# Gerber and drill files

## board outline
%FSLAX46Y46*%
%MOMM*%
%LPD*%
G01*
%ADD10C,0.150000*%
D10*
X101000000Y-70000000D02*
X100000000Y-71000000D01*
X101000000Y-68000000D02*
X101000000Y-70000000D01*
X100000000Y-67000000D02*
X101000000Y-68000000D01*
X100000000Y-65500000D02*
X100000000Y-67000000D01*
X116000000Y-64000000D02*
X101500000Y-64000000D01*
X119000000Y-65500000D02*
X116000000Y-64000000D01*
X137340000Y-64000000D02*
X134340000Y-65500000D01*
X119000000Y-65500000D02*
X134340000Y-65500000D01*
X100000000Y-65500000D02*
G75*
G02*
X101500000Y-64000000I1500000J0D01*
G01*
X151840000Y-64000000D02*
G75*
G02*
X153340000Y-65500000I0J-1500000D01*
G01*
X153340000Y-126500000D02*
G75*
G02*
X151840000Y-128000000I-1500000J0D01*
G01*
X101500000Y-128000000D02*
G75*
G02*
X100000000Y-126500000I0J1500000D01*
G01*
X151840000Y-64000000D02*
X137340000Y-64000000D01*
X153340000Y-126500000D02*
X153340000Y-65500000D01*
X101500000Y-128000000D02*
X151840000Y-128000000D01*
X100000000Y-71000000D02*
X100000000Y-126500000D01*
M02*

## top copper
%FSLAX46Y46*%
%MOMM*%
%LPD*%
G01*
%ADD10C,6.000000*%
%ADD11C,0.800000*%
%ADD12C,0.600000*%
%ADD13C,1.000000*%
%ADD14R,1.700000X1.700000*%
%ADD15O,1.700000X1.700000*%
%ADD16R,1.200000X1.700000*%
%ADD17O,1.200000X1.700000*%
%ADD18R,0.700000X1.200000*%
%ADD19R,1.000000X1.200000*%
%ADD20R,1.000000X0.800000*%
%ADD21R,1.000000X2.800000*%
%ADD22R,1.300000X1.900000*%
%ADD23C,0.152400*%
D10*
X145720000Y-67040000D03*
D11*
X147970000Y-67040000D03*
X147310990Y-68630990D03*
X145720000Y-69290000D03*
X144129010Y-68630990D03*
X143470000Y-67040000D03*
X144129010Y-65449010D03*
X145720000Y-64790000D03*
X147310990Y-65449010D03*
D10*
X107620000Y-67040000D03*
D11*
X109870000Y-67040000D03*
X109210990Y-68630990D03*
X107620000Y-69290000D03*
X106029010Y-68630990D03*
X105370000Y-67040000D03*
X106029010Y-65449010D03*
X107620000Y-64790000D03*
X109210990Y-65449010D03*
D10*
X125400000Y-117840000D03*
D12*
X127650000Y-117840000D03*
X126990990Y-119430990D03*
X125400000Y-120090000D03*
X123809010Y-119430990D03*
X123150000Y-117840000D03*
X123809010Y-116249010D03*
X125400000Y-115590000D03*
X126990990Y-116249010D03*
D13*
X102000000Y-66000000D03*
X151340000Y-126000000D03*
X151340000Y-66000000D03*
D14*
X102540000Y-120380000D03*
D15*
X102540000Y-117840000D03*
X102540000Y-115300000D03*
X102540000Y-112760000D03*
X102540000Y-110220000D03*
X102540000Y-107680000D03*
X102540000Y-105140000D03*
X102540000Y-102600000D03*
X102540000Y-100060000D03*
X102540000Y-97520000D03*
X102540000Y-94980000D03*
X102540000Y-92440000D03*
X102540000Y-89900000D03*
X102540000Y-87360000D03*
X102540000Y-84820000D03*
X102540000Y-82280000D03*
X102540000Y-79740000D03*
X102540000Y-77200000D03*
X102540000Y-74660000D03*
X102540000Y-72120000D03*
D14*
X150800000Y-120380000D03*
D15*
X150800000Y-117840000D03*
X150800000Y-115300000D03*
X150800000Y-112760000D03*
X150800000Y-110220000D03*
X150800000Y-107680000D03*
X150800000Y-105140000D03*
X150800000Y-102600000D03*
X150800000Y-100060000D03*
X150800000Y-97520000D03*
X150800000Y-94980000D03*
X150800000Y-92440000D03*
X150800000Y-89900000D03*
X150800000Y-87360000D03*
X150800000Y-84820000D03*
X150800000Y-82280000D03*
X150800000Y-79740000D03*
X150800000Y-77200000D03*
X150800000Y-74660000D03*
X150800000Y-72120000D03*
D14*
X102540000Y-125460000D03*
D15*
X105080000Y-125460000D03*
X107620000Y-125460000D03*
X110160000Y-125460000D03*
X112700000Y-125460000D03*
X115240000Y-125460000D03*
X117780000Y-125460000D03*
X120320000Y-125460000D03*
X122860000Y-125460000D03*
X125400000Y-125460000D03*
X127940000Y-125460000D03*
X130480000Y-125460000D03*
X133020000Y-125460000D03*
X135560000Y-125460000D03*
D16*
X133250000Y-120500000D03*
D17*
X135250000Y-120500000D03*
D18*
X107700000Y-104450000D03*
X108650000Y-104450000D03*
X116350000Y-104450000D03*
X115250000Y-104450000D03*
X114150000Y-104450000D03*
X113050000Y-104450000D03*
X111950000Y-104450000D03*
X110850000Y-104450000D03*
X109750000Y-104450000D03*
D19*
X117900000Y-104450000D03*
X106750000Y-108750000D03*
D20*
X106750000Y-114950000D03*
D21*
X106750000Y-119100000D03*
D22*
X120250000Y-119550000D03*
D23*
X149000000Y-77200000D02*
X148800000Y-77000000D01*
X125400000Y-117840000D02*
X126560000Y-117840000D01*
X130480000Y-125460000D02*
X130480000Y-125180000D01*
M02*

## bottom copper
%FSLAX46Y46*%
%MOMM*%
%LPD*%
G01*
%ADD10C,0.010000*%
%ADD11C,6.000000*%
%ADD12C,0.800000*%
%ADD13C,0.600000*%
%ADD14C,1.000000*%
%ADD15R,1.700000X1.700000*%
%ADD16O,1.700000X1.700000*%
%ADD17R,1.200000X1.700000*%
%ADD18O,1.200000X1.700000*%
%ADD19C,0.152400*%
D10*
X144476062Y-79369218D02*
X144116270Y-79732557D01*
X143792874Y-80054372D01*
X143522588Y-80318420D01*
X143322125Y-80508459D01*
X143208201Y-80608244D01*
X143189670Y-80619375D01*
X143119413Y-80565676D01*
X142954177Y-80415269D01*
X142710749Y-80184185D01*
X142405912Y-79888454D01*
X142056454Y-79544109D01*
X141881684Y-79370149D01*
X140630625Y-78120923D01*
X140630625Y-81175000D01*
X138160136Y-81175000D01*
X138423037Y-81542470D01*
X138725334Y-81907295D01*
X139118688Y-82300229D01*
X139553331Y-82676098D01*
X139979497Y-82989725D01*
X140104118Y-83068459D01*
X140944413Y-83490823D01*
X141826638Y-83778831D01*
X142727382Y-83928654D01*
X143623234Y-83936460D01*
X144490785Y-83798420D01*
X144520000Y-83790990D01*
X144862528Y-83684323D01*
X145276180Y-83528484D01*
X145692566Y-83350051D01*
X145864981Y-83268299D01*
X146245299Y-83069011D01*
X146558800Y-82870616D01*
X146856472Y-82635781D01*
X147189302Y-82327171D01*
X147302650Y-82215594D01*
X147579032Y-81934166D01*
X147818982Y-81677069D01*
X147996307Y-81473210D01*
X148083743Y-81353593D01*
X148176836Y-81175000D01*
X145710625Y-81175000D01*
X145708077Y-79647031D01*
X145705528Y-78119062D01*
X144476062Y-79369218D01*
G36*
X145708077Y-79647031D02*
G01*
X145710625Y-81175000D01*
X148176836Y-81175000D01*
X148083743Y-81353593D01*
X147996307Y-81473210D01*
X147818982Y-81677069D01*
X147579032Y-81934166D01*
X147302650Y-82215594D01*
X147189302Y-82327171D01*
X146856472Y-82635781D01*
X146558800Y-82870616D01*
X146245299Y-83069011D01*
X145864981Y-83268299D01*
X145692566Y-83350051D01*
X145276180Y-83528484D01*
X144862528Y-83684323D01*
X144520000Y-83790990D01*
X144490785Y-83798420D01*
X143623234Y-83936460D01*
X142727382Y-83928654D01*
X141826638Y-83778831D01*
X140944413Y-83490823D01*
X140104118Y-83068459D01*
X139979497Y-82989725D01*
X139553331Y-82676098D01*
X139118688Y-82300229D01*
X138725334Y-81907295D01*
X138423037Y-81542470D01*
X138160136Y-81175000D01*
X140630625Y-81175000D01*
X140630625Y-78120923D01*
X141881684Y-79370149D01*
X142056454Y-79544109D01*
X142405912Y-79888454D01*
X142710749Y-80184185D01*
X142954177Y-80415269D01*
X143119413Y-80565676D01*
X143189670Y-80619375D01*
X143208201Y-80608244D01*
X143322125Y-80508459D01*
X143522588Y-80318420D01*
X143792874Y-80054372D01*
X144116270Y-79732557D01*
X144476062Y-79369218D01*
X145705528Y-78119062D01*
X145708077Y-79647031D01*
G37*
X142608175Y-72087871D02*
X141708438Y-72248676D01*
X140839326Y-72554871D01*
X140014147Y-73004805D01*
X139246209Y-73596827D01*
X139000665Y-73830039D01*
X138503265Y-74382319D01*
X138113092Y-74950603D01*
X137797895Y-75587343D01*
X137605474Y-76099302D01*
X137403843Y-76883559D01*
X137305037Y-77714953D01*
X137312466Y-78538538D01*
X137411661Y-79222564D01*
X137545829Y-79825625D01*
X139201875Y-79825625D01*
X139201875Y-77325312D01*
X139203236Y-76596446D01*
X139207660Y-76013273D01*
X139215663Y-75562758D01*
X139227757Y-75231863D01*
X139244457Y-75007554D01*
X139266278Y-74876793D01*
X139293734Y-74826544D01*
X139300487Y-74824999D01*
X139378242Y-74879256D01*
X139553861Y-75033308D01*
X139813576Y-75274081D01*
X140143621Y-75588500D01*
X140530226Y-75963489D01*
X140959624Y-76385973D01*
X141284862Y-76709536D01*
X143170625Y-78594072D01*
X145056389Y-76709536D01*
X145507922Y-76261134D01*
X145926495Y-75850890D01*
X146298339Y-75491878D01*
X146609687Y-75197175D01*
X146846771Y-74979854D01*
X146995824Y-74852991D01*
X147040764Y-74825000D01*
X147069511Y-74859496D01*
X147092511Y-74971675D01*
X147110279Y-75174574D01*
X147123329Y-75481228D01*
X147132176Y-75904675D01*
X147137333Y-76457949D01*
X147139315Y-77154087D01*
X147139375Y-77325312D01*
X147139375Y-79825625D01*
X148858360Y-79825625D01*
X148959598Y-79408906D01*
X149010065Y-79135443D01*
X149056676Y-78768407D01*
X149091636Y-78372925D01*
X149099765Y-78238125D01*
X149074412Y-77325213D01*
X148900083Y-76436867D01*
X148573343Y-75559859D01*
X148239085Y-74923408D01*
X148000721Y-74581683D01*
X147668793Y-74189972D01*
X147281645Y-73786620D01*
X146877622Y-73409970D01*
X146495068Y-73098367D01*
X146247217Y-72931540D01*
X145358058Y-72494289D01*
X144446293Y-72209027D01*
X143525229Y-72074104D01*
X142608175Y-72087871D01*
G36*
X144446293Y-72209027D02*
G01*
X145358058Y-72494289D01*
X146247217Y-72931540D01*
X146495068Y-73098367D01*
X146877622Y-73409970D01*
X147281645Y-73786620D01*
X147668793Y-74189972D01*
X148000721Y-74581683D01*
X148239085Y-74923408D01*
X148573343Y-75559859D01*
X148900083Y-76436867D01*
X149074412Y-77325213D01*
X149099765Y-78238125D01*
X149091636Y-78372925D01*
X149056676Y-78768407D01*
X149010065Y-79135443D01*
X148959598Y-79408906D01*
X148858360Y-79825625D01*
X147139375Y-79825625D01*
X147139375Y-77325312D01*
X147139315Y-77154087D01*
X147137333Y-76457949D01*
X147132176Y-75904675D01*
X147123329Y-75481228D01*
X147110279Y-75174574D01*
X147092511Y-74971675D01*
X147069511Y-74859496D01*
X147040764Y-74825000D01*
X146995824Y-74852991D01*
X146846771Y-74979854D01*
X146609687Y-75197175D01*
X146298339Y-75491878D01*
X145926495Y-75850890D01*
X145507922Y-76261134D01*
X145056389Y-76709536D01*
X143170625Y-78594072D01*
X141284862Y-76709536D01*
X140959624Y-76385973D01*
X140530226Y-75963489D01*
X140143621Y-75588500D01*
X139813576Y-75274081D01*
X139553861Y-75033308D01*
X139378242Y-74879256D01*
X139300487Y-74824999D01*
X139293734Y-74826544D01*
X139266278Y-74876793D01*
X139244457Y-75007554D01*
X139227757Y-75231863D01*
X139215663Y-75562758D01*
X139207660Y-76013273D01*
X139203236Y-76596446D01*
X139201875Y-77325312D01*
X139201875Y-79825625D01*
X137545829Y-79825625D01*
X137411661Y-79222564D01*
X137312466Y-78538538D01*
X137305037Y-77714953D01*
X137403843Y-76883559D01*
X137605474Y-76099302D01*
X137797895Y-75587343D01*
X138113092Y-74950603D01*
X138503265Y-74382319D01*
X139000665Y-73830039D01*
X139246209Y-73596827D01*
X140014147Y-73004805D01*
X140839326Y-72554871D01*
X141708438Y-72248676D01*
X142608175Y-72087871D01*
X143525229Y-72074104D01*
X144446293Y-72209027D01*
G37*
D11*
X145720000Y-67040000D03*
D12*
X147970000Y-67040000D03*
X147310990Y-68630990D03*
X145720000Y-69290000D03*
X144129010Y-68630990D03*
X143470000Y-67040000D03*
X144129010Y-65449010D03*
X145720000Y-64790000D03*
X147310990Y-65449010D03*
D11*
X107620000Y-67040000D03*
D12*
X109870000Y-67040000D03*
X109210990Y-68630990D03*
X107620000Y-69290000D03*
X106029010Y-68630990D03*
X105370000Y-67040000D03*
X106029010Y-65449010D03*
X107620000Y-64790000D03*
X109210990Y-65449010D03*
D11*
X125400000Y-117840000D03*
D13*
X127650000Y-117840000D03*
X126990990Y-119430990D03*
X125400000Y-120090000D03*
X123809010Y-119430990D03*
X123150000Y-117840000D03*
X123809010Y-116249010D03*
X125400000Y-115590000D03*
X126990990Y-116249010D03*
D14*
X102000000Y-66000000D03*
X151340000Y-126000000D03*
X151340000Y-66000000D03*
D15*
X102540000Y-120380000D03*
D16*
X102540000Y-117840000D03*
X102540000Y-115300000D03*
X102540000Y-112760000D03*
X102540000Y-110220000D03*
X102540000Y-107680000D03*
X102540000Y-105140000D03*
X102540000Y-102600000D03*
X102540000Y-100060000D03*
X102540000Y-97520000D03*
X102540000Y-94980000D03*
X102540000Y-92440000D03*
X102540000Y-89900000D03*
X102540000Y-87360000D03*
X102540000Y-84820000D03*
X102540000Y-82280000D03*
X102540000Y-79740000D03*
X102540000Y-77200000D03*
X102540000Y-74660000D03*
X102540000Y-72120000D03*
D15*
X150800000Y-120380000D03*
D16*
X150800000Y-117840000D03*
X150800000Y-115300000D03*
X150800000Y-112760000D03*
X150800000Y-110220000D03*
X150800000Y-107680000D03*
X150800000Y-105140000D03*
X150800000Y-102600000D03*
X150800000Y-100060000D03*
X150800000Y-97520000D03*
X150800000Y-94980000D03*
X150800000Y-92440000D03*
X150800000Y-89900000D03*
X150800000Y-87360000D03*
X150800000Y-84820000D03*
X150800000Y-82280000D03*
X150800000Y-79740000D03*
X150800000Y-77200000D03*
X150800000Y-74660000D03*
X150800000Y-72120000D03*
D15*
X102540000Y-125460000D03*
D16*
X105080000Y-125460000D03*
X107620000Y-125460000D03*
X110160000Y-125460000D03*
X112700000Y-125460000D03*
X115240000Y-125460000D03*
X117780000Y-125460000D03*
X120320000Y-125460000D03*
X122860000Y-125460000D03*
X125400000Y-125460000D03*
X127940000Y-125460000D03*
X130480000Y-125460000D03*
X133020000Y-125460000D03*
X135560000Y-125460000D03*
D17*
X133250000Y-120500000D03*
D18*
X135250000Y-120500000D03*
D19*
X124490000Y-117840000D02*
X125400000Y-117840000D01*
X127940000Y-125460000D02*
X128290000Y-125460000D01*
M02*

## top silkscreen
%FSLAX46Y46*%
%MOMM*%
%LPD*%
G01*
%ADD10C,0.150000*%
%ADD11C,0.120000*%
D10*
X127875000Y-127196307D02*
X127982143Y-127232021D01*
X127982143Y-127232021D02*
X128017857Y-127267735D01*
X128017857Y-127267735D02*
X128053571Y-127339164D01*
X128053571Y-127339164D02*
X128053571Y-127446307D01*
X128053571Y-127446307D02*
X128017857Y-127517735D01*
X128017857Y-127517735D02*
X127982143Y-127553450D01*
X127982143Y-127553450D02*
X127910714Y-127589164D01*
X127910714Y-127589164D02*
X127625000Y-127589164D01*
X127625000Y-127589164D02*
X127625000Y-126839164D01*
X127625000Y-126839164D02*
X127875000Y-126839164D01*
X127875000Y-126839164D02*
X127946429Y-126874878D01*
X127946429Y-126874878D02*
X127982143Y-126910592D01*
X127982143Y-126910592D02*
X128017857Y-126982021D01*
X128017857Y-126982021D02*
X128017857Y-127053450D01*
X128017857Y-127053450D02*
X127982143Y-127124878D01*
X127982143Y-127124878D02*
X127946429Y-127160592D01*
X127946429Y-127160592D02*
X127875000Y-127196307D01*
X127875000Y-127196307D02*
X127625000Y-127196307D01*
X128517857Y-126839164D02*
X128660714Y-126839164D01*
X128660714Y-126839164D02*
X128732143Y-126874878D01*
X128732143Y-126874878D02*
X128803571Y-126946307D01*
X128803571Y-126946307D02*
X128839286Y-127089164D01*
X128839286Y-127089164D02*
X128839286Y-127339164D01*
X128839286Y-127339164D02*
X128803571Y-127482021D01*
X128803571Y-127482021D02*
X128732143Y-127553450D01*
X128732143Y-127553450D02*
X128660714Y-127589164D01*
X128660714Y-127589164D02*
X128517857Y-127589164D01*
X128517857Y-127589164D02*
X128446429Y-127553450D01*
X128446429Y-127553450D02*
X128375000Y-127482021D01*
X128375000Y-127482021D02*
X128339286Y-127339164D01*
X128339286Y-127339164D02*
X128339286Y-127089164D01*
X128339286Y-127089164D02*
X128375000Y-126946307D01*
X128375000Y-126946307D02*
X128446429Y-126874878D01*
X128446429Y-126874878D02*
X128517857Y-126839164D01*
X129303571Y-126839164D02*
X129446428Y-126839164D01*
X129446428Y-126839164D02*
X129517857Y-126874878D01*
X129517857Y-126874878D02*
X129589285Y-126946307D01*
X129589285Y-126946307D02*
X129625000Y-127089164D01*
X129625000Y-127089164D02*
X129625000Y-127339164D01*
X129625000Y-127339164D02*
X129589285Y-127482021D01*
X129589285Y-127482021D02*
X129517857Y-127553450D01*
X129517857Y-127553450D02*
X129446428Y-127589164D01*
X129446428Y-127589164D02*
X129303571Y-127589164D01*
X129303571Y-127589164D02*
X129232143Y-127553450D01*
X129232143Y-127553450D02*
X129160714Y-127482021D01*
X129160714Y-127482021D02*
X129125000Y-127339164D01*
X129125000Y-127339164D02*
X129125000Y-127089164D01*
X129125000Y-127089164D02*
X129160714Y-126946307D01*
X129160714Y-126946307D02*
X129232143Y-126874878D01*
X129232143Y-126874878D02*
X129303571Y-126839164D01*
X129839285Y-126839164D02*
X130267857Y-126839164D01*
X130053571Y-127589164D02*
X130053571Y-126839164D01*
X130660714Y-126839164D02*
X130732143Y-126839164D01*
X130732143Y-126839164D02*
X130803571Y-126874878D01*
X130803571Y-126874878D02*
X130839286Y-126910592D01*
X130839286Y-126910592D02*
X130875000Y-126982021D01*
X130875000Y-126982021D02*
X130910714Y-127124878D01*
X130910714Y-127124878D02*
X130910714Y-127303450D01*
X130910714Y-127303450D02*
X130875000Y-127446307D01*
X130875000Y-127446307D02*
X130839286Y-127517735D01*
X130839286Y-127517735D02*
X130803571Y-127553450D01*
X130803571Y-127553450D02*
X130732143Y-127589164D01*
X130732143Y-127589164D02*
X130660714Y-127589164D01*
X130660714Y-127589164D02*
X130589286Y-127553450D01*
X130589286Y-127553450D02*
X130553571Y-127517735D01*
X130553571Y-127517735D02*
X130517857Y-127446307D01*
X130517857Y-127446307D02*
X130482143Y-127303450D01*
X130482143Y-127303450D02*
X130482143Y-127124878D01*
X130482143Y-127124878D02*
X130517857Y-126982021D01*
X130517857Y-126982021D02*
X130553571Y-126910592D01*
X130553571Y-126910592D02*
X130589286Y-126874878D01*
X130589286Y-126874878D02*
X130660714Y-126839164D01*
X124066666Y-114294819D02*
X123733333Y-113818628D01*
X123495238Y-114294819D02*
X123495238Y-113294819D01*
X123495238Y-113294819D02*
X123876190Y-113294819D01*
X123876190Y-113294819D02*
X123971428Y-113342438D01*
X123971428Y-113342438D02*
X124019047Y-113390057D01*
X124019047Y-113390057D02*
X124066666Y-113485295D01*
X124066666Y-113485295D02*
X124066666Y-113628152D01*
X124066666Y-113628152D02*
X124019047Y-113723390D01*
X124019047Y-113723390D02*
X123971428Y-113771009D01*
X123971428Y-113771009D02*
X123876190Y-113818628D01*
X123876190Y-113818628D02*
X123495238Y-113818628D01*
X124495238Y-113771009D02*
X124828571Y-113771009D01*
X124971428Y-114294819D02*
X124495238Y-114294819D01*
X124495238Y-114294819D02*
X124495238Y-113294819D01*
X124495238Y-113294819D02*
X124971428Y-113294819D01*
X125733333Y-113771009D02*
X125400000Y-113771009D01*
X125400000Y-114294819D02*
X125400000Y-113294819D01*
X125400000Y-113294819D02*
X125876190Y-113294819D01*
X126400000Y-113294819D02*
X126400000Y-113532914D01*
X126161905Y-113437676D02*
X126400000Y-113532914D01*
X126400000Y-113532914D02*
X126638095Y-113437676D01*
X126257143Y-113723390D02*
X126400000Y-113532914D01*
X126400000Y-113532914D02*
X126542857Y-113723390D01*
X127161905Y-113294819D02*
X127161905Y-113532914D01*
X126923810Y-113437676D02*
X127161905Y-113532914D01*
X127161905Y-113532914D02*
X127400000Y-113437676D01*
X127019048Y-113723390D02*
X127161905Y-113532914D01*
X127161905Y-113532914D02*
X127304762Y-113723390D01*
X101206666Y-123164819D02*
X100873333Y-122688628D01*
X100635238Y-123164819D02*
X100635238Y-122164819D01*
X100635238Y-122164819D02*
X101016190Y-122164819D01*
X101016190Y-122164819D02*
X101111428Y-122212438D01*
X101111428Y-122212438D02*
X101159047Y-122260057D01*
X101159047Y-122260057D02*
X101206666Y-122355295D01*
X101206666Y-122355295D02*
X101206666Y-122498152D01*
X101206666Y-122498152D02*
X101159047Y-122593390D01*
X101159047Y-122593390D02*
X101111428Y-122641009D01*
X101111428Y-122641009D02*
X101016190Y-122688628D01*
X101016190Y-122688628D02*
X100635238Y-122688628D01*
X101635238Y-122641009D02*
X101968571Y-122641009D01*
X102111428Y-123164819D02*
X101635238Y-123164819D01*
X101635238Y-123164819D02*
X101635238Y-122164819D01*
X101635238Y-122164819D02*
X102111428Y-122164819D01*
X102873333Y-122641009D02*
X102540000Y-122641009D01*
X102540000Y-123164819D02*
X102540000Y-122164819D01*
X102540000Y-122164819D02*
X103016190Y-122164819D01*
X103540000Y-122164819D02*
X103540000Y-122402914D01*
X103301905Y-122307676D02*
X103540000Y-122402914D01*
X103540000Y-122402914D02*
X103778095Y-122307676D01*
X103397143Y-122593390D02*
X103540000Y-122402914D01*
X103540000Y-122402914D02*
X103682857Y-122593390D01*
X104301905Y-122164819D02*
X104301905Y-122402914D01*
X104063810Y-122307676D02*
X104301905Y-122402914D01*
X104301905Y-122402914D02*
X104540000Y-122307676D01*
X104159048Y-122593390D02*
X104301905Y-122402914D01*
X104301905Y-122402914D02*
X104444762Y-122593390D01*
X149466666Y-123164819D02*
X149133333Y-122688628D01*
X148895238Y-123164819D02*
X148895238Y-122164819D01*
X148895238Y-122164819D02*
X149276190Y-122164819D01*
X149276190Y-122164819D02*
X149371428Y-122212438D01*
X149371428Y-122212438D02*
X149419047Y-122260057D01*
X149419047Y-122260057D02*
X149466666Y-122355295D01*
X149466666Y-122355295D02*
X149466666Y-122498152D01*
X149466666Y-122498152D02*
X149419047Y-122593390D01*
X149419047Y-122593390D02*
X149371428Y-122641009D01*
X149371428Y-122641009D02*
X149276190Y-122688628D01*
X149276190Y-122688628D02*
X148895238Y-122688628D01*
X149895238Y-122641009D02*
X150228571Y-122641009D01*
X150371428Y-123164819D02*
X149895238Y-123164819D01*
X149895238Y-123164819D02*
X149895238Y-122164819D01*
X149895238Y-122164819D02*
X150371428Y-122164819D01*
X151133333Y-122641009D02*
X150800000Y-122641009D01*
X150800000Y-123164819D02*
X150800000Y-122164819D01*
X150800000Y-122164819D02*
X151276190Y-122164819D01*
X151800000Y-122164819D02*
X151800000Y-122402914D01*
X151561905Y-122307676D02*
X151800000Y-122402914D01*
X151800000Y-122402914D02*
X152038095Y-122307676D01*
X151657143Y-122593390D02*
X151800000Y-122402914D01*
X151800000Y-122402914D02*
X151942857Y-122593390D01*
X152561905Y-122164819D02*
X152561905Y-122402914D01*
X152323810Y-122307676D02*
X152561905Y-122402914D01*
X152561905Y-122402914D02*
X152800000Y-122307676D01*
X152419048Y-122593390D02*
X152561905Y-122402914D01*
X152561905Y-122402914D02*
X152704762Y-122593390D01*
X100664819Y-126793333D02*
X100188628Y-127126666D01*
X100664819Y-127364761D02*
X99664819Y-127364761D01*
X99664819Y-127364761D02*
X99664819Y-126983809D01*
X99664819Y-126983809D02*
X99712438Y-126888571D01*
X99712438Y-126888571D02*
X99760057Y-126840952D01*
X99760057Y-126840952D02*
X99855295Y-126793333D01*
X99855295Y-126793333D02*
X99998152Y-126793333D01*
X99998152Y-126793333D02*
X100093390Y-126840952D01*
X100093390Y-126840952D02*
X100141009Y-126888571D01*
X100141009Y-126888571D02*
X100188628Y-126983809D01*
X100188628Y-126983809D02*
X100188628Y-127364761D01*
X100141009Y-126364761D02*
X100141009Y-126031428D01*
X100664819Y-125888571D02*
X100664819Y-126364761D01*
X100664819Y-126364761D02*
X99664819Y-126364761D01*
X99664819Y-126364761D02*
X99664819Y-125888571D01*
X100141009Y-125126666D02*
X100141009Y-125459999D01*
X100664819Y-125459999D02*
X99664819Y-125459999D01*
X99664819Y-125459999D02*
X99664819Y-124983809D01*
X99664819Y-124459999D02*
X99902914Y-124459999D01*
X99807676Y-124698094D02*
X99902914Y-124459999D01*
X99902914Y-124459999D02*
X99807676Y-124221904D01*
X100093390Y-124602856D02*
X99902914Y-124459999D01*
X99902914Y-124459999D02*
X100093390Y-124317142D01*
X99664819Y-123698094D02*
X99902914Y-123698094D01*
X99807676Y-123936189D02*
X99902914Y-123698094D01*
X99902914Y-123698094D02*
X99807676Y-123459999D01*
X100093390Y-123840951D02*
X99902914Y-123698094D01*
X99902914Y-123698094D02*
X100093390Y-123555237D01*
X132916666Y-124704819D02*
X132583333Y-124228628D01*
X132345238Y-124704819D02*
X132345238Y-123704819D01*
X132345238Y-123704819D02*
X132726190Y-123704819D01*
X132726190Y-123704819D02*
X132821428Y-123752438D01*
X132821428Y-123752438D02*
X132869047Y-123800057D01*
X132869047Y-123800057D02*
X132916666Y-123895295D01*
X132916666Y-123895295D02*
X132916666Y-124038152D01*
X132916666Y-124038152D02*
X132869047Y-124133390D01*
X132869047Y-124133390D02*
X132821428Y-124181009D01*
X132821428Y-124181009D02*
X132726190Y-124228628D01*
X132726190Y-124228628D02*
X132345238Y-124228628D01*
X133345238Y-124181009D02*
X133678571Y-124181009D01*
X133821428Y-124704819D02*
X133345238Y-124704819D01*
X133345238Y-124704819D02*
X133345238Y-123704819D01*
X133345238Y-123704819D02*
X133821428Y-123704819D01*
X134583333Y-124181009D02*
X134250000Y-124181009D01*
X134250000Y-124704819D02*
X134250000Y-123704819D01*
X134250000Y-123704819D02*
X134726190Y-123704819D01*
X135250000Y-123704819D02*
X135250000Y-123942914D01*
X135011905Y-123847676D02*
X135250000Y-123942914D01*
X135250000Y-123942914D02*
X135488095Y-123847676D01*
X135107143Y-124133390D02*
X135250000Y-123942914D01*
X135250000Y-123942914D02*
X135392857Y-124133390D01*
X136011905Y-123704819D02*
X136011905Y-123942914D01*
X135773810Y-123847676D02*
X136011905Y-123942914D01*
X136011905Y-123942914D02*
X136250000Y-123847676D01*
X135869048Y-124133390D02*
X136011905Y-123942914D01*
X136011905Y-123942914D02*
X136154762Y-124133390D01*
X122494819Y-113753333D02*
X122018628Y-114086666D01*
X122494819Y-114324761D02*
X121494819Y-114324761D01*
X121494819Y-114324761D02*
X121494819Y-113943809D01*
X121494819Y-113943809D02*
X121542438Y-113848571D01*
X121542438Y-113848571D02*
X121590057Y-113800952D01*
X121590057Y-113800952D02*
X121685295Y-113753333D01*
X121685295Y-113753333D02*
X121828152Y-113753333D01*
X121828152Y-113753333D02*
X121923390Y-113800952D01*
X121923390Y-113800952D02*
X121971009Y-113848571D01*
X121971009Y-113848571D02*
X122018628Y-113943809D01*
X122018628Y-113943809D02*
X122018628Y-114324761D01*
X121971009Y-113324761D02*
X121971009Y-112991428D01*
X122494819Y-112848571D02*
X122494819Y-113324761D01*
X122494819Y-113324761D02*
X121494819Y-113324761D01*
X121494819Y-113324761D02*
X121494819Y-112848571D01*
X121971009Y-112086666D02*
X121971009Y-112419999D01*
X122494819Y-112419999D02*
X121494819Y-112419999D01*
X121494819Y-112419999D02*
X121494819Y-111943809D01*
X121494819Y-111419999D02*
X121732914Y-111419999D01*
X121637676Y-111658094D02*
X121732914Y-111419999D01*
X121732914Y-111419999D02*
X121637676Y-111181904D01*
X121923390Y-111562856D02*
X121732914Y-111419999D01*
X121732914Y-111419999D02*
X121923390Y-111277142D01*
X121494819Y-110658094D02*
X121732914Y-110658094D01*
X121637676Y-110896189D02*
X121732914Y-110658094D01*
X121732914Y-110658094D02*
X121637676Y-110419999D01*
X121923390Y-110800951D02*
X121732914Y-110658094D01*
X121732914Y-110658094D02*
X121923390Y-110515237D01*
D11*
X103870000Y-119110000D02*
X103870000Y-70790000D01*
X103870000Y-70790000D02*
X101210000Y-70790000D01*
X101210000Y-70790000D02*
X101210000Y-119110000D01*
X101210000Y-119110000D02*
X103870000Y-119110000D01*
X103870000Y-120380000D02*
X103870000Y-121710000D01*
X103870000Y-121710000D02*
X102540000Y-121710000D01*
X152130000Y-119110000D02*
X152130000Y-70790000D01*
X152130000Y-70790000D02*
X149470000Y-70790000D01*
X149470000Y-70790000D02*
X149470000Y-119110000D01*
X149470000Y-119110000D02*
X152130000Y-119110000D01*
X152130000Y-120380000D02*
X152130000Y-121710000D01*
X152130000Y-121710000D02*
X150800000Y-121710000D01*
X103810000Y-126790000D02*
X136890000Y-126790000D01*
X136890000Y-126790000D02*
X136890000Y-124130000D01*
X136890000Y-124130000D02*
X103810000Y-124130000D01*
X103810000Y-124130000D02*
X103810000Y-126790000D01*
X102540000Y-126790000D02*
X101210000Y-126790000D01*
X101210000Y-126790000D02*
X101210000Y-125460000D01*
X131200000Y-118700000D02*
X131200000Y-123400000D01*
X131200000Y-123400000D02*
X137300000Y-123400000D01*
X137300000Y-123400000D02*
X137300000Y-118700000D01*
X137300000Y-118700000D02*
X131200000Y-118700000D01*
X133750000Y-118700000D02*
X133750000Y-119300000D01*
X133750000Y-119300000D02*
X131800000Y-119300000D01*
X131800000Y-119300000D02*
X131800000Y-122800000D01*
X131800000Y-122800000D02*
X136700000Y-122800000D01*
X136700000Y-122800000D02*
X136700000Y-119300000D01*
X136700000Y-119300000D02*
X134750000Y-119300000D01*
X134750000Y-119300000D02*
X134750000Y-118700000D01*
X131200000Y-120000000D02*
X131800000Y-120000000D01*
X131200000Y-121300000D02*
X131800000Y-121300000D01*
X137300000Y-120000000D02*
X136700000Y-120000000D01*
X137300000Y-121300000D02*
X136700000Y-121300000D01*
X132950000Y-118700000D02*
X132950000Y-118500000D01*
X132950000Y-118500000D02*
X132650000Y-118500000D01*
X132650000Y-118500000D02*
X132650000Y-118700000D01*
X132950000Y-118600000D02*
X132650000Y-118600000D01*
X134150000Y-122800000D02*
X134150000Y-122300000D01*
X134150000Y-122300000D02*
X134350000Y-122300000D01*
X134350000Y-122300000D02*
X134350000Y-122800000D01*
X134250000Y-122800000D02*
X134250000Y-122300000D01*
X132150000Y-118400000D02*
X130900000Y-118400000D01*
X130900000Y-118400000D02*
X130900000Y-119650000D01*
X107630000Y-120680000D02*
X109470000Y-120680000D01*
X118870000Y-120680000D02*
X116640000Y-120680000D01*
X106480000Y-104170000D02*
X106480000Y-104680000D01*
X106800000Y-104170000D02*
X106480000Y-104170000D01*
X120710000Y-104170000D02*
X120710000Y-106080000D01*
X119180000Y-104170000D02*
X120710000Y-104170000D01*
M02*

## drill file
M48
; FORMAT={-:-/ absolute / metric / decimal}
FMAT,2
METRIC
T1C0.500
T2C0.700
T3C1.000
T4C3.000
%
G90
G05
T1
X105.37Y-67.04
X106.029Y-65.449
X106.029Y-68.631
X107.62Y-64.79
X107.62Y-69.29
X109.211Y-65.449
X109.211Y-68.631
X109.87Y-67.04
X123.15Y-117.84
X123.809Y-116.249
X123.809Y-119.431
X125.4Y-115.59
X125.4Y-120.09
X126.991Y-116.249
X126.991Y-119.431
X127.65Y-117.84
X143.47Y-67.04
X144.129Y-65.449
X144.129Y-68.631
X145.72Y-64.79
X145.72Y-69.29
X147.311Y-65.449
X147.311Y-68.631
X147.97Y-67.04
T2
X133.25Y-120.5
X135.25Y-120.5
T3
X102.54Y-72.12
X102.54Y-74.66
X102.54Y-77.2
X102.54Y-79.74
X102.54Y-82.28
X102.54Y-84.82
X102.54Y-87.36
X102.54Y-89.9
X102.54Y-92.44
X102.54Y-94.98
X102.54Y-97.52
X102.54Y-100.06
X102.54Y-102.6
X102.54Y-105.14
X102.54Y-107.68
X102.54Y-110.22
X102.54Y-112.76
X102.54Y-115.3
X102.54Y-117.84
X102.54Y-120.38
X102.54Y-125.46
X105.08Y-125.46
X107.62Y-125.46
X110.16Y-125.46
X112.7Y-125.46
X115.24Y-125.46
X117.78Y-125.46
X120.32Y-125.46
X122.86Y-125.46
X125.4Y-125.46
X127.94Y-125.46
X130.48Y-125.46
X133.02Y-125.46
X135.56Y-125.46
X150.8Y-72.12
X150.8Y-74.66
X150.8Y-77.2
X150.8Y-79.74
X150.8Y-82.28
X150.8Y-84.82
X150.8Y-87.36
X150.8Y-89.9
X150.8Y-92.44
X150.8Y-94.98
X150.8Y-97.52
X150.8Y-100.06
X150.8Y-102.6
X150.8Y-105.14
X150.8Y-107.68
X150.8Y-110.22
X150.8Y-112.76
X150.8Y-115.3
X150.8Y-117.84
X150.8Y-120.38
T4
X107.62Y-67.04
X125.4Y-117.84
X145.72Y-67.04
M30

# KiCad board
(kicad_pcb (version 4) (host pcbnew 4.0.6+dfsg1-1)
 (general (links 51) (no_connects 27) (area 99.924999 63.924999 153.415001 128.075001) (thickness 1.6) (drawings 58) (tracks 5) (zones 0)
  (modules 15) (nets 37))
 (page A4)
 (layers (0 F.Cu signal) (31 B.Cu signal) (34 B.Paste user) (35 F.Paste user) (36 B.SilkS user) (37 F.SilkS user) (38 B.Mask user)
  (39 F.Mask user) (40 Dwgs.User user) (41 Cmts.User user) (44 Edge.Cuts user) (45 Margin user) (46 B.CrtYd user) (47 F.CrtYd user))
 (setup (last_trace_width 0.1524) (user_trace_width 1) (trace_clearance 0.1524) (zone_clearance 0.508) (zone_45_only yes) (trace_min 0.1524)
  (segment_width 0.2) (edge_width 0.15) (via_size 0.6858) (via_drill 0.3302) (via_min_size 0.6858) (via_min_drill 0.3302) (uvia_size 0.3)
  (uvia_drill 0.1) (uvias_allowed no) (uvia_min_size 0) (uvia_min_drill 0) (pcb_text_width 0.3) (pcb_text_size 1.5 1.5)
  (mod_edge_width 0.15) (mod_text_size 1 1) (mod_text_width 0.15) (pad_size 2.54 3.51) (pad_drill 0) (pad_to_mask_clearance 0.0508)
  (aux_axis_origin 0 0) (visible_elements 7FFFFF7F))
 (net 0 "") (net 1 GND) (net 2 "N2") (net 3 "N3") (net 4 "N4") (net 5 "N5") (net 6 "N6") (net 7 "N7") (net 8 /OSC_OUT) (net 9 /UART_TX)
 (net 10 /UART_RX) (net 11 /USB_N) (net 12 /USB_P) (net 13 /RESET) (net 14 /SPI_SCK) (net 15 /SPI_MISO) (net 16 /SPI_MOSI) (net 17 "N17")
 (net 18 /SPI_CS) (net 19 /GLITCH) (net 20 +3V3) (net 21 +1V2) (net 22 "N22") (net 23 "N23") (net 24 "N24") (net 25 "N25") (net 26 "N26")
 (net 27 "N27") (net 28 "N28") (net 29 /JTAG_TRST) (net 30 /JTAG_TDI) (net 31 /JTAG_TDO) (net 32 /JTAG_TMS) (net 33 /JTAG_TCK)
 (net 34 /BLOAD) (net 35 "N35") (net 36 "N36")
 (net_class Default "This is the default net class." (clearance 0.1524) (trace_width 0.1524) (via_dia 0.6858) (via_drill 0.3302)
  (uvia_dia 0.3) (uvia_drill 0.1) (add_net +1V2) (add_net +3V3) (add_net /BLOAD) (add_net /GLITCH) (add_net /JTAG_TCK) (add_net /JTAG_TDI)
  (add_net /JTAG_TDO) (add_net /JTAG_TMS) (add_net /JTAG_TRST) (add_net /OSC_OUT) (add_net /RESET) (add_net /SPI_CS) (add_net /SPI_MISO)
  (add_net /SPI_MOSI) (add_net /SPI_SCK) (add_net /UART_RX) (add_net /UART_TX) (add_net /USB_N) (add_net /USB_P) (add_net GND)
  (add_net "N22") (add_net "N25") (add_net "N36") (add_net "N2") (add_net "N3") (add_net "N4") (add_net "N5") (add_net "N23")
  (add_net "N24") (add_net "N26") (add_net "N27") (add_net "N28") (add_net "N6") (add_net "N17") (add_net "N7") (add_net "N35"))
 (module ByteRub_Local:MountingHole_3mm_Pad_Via (layer F.Cu) (at 145.72 67.04)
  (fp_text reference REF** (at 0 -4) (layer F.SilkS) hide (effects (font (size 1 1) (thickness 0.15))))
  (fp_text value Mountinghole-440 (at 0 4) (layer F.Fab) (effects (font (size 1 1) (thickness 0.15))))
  (pad 1 thru_hole circle (at 0 0) (size 6 6) (drill 3) (layers *.Cu *.Mask) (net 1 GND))
  (pad 1 thru_hole circle (at 2.25 0) (size 0.8 0.8) (drill 0.5) (layers *.Cu *.Mask) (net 1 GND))
  (pad 1 thru_hole circle (at 1.59099 1.59099) (size 0.8 0.8) (drill 0.5) (layers *.Cu *.Mask) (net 1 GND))
  (pad 1 thru_hole circle (at 0 2.25) (size 0.8 0.8) (drill 0.5) (layers *.Cu *.Mask) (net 1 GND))
  (pad 1 thru_hole circle (at -1.59099 1.59099) (size 0.8 0.8) (drill 0.5) (layers *.Cu *.Mask) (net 1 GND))
  (pad 1 thru_hole circle (at -2.25 0) (size 0.8 0.8) (drill 0.5) (layers *.Cu *.Mask) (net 1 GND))
  (pad 1 thru_hole circle (at -1.59099 -1.59099) (size 0.8 0.8) (drill 0.5) (layers *.Cu *.Mask) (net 1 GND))
  (pad 1 thru_hole circle (at 0 -2.25) (size 0.8 0.8) (drill 0.5) (layers *.Cu *.Mask) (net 1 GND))
  (pad 1 thru_hole circle (at 1.59099 -1.59099) (size 0.8 0.8) (drill 0.5) (layers *.Cu *.Mask) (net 1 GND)))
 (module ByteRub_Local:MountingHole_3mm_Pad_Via (layer F.Cu) (at 107.62 67.04)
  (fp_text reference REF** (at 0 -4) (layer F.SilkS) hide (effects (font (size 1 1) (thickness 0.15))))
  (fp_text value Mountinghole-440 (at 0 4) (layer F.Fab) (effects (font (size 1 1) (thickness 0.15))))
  (pad 1 thru_hole circle (at 0 0) (size 6 6) (drill 3) (layers *.Cu *.Mask) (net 1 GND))
  (pad 1 thru_hole circle (at 2.25 0) (size 0.8 0.8) (drill 0.5) (layers *.Cu *.Mask) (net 1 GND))
  (pad 1 thru_hole circle (at 1.59099 1.59099) (size 0.8 0.8) (drill 0.5) (layers *.Cu *.Mask) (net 1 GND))
  (pad 1 thru_hole circle (at 0 2.25) (size 0.8 0.8) (drill 0.5) (layers *.Cu *.Mask) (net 1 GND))
  (pad 1 thru_hole circle (at -1.59099 1.59099) (size 0.8 0.8) (drill 0.5) (layers *.Cu *.Mask) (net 1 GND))
  (pad 1 thru_hole circle (at -2.25 0) (size 0.8 0.8) (drill 0.5) (layers *.Cu *.Mask) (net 1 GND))
  (pad 1 thru_hole circle (at -1.59099 -1.59099) (size 0.8 0.8) (drill 0.5) (layers *.Cu *.Mask) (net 1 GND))
  (pad 1 thru_hole circle (at 0 -2.25) (size 0.8 0.8) (drill 0.5) (layers *.Cu *.Mask) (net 1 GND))
  (pad 1 thru_hole circle (at 1.59099 -1.59099) (size 0.8 0.8) (drill 0.5) (layers *.Cu *.Mask) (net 1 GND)))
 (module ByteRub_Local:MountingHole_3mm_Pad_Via (layer F.Cu) (at 125.4 117.84)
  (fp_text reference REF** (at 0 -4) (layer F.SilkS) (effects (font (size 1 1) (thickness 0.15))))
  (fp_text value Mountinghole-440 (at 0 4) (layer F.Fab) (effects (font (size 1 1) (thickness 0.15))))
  (pad 1 thru_hole circle (at 0 0) (size 6 6) (drill 3) (layers *.Cu *.Mask) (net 1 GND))
  (pad 1 thru_hole circle (at 2.25 0) (size 0.6 0.6) (drill 0.5) (layers *.Cu *.Mask) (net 1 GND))
  (pad 1 thru_hole circle (at 1.59099 1.59099) (size 0.6 0.6) (drill 0.5) (layers *.Cu *.Mask) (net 1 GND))
  (pad 1 thru_hole circle (at 0 2.25) (size 0.6 0.6) (drill 0.5) (layers *.Cu *.Mask) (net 1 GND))
  (pad 1 thru_hole circle (at -1.59099 1.59099) (size 0.6 0.6) (drill 0.5) (layers *.Cu *.Mask) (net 1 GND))
  (pad 1 thru_hole circle (at -2.25 0) (size 0.6 0.6) (drill 0.5) (layers *.Cu *.Mask) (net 1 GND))
  (pad 1 thru_hole circle (at -1.59099 -1.59099) (size 0.6 0.6) (drill 0.5) (layers *.Cu *.Mask) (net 1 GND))
  (pad 1 thru_hole circle (at 0 -2.25) (size 0.6 0.6) (drill 0.5) (layers *.Cu *.Mask) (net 1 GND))
  (pad 1 thru_hole circle (at 1.59099 -1.59099) (size 0.6 0.6) (drill 0.5) (layers *.Cu *.Mask) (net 1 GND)))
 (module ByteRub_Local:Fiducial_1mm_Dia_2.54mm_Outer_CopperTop (layer F.Cu) (at 102 66)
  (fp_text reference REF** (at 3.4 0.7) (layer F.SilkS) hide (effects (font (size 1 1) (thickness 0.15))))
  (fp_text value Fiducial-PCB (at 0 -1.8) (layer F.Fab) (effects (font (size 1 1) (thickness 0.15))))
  (pad ~ smd circle (at 0 0) (size 1 1) (layers F.Cu F.Mask) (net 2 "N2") (solder_mask_margin 0.77) (clearance 0.77)))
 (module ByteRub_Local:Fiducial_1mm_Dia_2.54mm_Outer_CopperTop (layer F.Cu) (at 151.34 126)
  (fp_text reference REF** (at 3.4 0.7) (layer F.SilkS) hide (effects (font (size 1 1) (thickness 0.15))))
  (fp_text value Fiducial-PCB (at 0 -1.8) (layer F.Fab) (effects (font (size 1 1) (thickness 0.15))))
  (pad ~ smd circle (at 0 0) (size 1 1) (layers F.Cu F.Mask) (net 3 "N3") (solder_mask_margin 0.77) (clearance 0.77)))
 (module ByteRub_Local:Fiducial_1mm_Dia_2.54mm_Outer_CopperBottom (layer F.Cu) (at 102 66)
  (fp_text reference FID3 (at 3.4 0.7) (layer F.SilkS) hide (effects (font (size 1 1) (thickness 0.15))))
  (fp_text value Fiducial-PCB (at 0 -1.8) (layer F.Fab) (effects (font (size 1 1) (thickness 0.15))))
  (pad ~ smd circle (at 0 0) (size 1 1) (layers B.Cu B.Mask) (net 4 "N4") (solder_mask_margin 0.77) (clearance 0.77)))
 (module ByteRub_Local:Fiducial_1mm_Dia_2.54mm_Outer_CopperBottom (layer F.Cu) (at 151.34 126)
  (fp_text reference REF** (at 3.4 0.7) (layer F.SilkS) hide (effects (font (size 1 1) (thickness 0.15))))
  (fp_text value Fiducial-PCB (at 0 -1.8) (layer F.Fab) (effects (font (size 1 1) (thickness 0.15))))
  (pad ~ smd circle (at 0 0) (size 1 1) (layers B.Cu B.Mask) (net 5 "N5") (solder_mask_margin 0.77) (clearance 0.77)))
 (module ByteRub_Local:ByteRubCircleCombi (layer B.Cu) (at 143.25 78 180)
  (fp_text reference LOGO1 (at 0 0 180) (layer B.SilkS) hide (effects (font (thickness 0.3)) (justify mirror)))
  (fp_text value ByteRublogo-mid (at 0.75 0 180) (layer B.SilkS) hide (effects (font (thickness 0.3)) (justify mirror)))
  (fp_poly
   (pts (xy -1.226062 -1.369218) (xy -0.86627 -1.732557) (xy -0.542874 -2.054372) (xy -0.272588 -2.31842) (xy -0.072125 -2.508459)
    (xy 0.041799 -2.608244) (xy 0.06033 -2.619375) (xy 0.130587 -2.565676) (xy 0.295823 -2.415269) (xy 0.539251 -2.184185)
    (xy 0.844088 -1.888454) (xy 1.193546 -1.544109) (xy 1.368316 -1.370149) (xy 2.619375 -0.120923) (xy 2.619375 -3.175)
    (xy 5.089864 -3.175) (xy 4.826963 -3.54247) (xy 4.524666 -3.907295) (xy 4.131312 -4.300229) (xy 3.696669 -4.676098)
    (xy 3.270503 -4.989725) (xy 3.145882 -5.068459) (xy 2.305587 -5.490823) (xy 1.423362 -5.778831) (xy 0.522618 -5.928654)
    (xy -0.373234 -5.93646) (xy -1.240785 -5.79842) (xy -1.27 -5.79099) (xy -1.612528 -5.684323) (xy -2.02618 -5.528484)
    (xy -2.442566 -5.350051) (xy -2.614981 -5.268299) (xy -2.995299 -5.069011) (xy -3.3088 -4.870616) (xy -3.606472 -4.635781)
    (xy -3.939302 -4.327171) (xy -4.05265 -4.215594) (xy -4.329032 -3.934166) (xy -4.568982 -3.677069) (xy -4.746307 -3.47321)
    (xy -4.833743 -3.353593) (xy -4.926836 -3.175) (xy -2.460625 -3.175) (xy -2.458077 -1.647031) (xy -2.455528 -0.119062)
    (xy -1.226062 -1.369218))
   (layer B.Cu) (width 0.01))
  (fp_poly
   (pts (xy 0.641825 5.912129) (xy 1.541562 5.751324) (xy 2.410674 5.445129) (xy 3.235853 4.995195) (xy 4.003791 4.403173)
    (xy 4.249335 4.169961) (xy 4.746735 3.617681) (xy 5.136908 3.049397) (xy 5.452105 2.412657) (xy 5.644526 1.900698)
    (xy 5.846157 1.116441) (xy 5.944963 0.285047) (xy 5.937534 -0.538538) (xy 5.838339 -1.222564) (xy 5.704171 -1.825625)
    (xy 4.048125 -1.825625) (xy 4.048125 0.674688) (xy 4.046764 1.403554) (xy 4.04234 1.986727) (xy 4.034337 2.437242)
    (xy 4.022243 2.768137) (xy 4.005543 2.992446) (xy 3.983722 3.123207) (xy 3.956266 3.173456) (xy 3.949513 3.175001)
    (xy 3.871758 3.120744) (xy 3.696139 2.966692) (xy 3.436424 2.725919) (xy 3.106379 2.4115) (xy 2.719774 2.036511) (xy 2.290376 1.614027)
    (xy 1.965138 1.290464) (xy 0.079375 -0.594072) (xy -1.806389 1.290464) (xy -2.257922 1.738866) (xy -2.676495 2.14911)
    (xy -3.048339 2.508122) (xy -3.359687 2.802825) (xy -3.596771 3.020146) (xy -3.745824 3.147009) (xy -3.790764 3.175)
    (xy -3.819511 3.140504) (xy -3.842511 3.028325) (xy -3.860279 2.825426) (xy -3.873329 2.518772) (xy -3.882176 2.095325)
    (xy -3.887333 1.542051) (xy -3.889315 0.845913) (xy -3.889375 0.674688) (xy -3.889375 -1.825625) (xy -5.60836 -1.825625)
    (xy -5.709598 -1.408906) (xy -5.760065 -1.135443) (xy -5.806676 -0.768407) (xy -5.841636 -0.372925) (xy -5.849765 -0.238125)
    (xy -5.824412 0.674787) (xy -5.650083 1.563133) (xy -5.323343 2.440141) (xy -4.989085 3.076592) (xy -4.750721 3.418317)
    (xy -4.418793 3.810028) (xy -4.031645 4.21338) (xy -3.627622 4.59003) (xy -3.245068 4.901633) (xy -2.997217 5.06846)
    (xy -2.108058 5.505711) (xy -1.196293 5.790973) (xy -0.275229 5.925896) (xy 0.641825 5.912129))
   (layer B.Cu) (width 0.01)))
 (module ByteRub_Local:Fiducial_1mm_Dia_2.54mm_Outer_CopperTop (layer B.Cu) (at 151.34 66)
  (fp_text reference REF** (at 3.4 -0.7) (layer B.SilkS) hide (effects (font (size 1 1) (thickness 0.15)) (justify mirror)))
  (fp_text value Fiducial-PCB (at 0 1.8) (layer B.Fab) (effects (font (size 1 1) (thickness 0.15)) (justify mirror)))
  (pad ~ smd circle (at 0 0) (size 1 1) (layers B.Cu B.Mask) (solder_mask_margin 0.77) (clearance 0.77)))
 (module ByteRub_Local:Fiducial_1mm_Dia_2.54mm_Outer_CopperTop (layer F.Cu) (at 151.34 66)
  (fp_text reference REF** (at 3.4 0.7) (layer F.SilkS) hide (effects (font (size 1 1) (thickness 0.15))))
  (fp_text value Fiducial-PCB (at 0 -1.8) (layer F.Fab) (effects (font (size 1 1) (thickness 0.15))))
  (pad ~ smd circle (at 0 0) (size 1 1) (layers F.Cu F.Mask) (solder_mask_margin 0.77) (clearance 0.77)))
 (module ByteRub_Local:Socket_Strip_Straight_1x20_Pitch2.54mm (layer F.Cu) (at 102.54 120.38 180)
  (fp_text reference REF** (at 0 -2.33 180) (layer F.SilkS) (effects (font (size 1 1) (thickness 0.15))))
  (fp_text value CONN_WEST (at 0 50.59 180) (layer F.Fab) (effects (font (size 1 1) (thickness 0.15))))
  (fp_line (start -1.33 1.27) (end -1.33 49.59) (layer F.SilkS) (width 0.12))
  (fp_line (start -1.33 49.59) (end 1.33 49.59) (layer F.SilkS) (width 0.12))
  (fp_line (start 1.33 49.59) (end 1.33 1.27) (layer F.SilkS) (width 0.12))
  (fp_line (start 1.33 1.27) (end -1.33 1.27) (layer F.SilkS) (width 0.12))
  (fp_line (start -1.33 0) (end -1.33 -1.33) (layer F.SilkS) (width 0.12))
  (fp_line (start -1.33 -1.33) (end 0 -1.33) (layer F.SilkS) (width 0.12))
  (pad 1 thru_hole rect (at 0 0 180) (size 1.7 1.7) (drill 1) (layers *.Cu *.Mask) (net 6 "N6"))
  (pad 2 thru_hole oval (at 0 2.54 180) (size 1.7 1.7) (drill 1) (layers *.Cu *.Mask) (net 1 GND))
  (pad 3 thru_hole oval (at 0 5.08 180) (size 1.7 1.7) (drill 1) (layers *.Cu *.Mask) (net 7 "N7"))
  (pad 4 thru_hole oval (at 0 7.62 180) (size 1.7 1.7) (drill 1) (layers *.Cu *.Mask) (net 1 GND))
  (pad 5 thru_hole oval (at 0 10.16 180) (size 1.7 1.7) (drill 1) (layers *.Cu *.Mask) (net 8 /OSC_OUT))
  (pad 6 thru_hole oval (at 0 12.7 180) (size 1.7 1.7) (drill 1) (layers *.Cu *.Mask) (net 1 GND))
  (pad 7 thru_hole oval (at 0 15.24 180) (size 1.7 1.7) (drill 1) (layers *.Cu *.Mask) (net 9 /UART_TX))
  (pad 8 thru_hole oval (at 0 17.78 180) (size 1.7 1.7) (drill 1) (layers *.Cu *.Mask) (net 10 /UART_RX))
  (pad 9 thru_hole oval (at 0 20.32 180) (size 1.7 1.7) (drill 1) (layers *.Cu *.Mask) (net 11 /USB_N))
  (pad 10 thru_hole oval (at 0 22.86 180) (size 1.7 1.7) (drill 1) (layers *.Cu *.Mask) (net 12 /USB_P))
  (pad 11 thru_hole oval (at 0 25.4 180) (size 1.7 1.7) (drill 1) (layers *.Cu *.Mask) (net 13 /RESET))
  (pad 12 thru_hole oval (at 0 27.94 180) (size 1.7 1.7) (drill 1) (layers *.Cu *.Mask) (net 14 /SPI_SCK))
  (pad 13 thru_hole oval (at 0 30.48 180) (size 1.7 1.7) (drill 1) (layers *.Cu *.Mask) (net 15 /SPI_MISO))
  (pad 14 thru_hole oval (at 0 33.02 180) (size 1.7 1.7) (drill 1) (layers *.Cu *.Mask) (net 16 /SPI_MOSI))
  (pad 15 thru_hole oval (at 0 35.56 180) (size 1.7 1.7) (drill 1) (layers *.Cu *.Mask) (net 1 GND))
  (pad 16 thru_hole oval (at 0 38.1 180) (size 1.7 1.7) (drill 1) (layers *.Cu *.Mask) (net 1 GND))
  (pad 17 thru_hole oval (at 0 40.64 180) (size 1.7 1.7) (drill 1) (layers *.Cu *.Mask) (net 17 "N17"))
  (pad 18 thru_hole oval (at 0 43.18 180) (size 1.7 1.7) (drill 1) (layers *.Cu *.Mask) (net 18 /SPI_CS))
  (pad 19 thru_hole oval (at 0 45.72 180) (size 1.7 1.7) (drill 1) (layers *.Cu *.Mask) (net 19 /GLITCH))
  (pad 20 thru_hole oval (at 0 48.26 180) (size 1.7 1.7) (drill 1) (layers *.Cu *.Mask) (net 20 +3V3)))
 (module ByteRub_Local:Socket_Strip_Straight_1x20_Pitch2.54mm (layer F.Cu) (at 150.8 120.38 180)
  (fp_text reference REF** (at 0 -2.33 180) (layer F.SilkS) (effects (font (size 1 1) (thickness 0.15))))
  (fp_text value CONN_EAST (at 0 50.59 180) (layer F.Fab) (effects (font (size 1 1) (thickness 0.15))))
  (fp_line (start -1.33 1.27) (end -1.33 49.59) (layer F.SilkS) (width 0.12))
  (fp_line (start -1.33 49.59) (end 1.33 49.59) (layer F.SilkS) (width 0.12))
  (fp_line (start 1.33 49.59) (end 1.33 1.27) (layer F.SilkS) (width 0.12))
  (fp_line (start 1.33 1.27) (end -1.33 1.27) (layer F.SilkS) (width 0.12))
  (fp_line (start -1.33 0) (end -1.33 -1.33) (layer F.SilkS) (width 0.12))
  (fp_line (start -1.33 -1.33) (end 0 -1.33) (layer F.SilkS) (width 0.12))
  (pad 1 thru_hole rect (at 0 0 180) (size 1.7 1.7) (drill 1) (layers *.Cu *.Mask) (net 1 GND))
  (pad 2 thru_hole oval (at 0 2.54 180) (size 1.7 1.7) (drill 1) (layers *.Cu *.Mask) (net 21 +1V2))
  (pad 3 thru_hole oval (at 0 5.08 180) (size 1.7 1.7) (drill 1) (layers *.Cu *.Mask) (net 21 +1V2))
  (pad 4 thru_hole oval (at 0 7.62 180) (size 1.7 1.7) (drill 1) (layers *.Cu *.Mask) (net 1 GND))
  (pad 5 thru_hole oval (at 0 10.16 180) (size 1.7 1.7) (drill 1) (layers *.Cu *.Mask) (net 21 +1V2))
  (pad 6 thru_hole oval (at 0 12.7 180) (size 1.7 1.7) (drill 1) (layers *.Cu *.Mask) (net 21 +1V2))
  (pad 7 thru_hole oval (at 0 15.24 180) (size 1.7 1.7) (drill 1) (layers *.Cu *.Mask) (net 1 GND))
  (pad 8 thru_hole oval (at 0 17.78 180) (size 1.7 1.7) (drill 1) (layers *.Cu *.Mask) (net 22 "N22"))
  (pad 9 thru_hole oval (at 0 20.32 180) (size 1.7 1.7) (drill 1) (layers *.Cu *.Mask) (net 1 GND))
  (pad 10 thru_hole oval (at 0 22.86 180) (size 1.7 1.7) (drill 1) (layers *.Cu *.Mask) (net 1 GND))
  (pad 11 thru_hole oval (at 0 25.4 180) (size 1.7 1.7) (drill 1) (layers *.Cu *.Mask) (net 22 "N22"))
  (pad 12 thru_hole oval (at 0 27.94 180) (size 1.7 1.7) (drill 1) (layers *.Cu *.Mask) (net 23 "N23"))
  (pad 13 thru_hole oval (at 0 30.48 180) (size 1.7 1.7) (drill 1) (layers *.Cu *.Mask) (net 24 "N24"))
  (pad 14 thru_hole oval (at 0 33.02 180) (size 1.7 1.7) (drill 1) (layers *.Cu *.Mask) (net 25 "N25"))
  (pad 15 thru_hole oval (at 0 35.56 180) (size 1.7 1.7) (drill 1) (layers *.Cu *.Mask) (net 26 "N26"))
  (pad 16 thru_hole oval (at 0 38.1 180) (size 1.7 1.7) (drill 1) (layers *.Cu *.Mask) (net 1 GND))
  (pad 17 thru_hole oval (at 0 40.64 180) (size 1.7 1.7) (drill 1) (layers *.Cu *.Mask) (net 1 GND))
  (pad 18 thru_hole oval (at 0 43.18 180) (size 1.7 1.7) (drill 1) (layers *.Cu *.Mask) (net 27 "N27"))
  (pad 19 thru_hole oval (at 0 45.72 180) (size 1.7 1.7) (drill 1) (layers *.Cu *.Mask) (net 1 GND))
  (pad 20 thru_hole oval (at 0 48.26 180) (size 1.7 1.7) (drill 1) (layers *.Cu *.Mask) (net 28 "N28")))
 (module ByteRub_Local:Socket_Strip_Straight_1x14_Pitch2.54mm (layer F.Cu) (at 102.54 125.46 90)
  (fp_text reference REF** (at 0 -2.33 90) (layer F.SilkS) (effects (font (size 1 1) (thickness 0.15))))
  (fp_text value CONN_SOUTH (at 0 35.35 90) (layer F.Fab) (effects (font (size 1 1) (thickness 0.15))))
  (fp_line (start -1.33 1.27) (end -1.33 34.35) (layer F.SilkS) (width 0.12))
  (fp_line (start -1.33 34.35) (end 1.33 34.35) (layer F.SilkS) (width 0.12))
  (fp_line (start 1.33 34.35) (end 1.33 1.27) (layer F.SilkS) (width 0.12))
  (fp_line (start 1.33 1.27) (end -1.33 1.27) (layer F.SilkS) (width 0.12))
  (fp_line (start -1.33 0) (end -1.33 -1.33) (layer F.SilkS) (width 0.12))
  (fp_line (start -1.33 -1.33) (end 0 -1.33) (layer F.SilkS) (width 0.12))
  (pad 1 thru_hole rect (at 0 0 90) (size 1.7 1.7) (drill 1) (layers *.Cu *.Mask) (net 1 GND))
  (pad 2 thru_hole oval (at 0 2.54 90) (size 1.7 1.7) (drill 1) (layers *.Cu *.Mask) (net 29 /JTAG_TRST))
  (pad 3 thru_hole oval (at 0 5.08 90) (size 1.7 1.7) (drill 1) (layers *.Cu *.Mask) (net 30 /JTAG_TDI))
  (pad 4 thru_hole oval (at 0 7.62 90) (size 1.7 1.7) (drill 1) (layers *.Cu *.Mask) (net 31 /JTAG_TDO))
  (pad 5 thru_hole oval (at 0 10.16 90) (size 1.7 1.7) (drill 1) (layers *.Cu *.Mask) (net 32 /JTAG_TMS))
  (pad 6 thru_hole oval (at 0 12.7 90) (size 1.7 1.7) (drill 1) (layers *.Cu *.Mask) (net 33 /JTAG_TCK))
  (pad 7 thru_hole oval (at 0 15.24 90) (size 1.7 1.7) (drill 1) (layers *.Cu *.Mask) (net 20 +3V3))
  (pad 8 thru_hole oval (at 0 17.78 90) (size 1.7 1.7) (drill 1) (layers *.Cu *.Mask) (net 13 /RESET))
  (pad 9 thru_hole oval (at 0 20.32 90) (size 1.7 1.7) (drill 1) (layers *.Cu *.Mask) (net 1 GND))
  (pad 10 thru_hole oval (at 0 22.86 90) (size 1.7 1.7) (drill 1) (layers *.Cu *.Mask) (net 1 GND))
  (pad 11 thru_hole oval (at 0 25.4 90) (size 1.7 1.7) (drill 1) (layers *.Cu *.Mask) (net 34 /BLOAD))
  (pad 12 thru_hole oval (at 0 27.94 90) (size 1.7 1.7) (drill 1) (layers *.Cu *.Mask) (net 20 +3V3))
  (pad 13 thru_hole oval (at 0 30.48 90) (size 1.7 1.7) (drill 1) (layers *.Cu *.Mask) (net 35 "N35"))
  (pad 14 thru_hole oval (at 0 33.02 90) (size 1.7 1.7) (drill 1) (layers *.Cu *.Mask) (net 20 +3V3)))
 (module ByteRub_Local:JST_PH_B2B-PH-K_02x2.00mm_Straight (layer F.Cu) (at 133.25 120.5)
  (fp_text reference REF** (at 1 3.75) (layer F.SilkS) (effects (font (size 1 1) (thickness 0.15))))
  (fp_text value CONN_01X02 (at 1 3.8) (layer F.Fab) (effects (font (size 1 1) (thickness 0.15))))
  (fp_line (start -2.05 -1.8) (end -2.05 2.9) (layer F.SilkS) (width 0.12))
  (fp_line (start -2.05 2.9) (end 4.05 2.9) (layer F.SilkS) (width 0.12))
  (fp_line (start 4.05 2.9) (end 4.05 -1.8) (layer F.SilkS) (width 0.12))
  (fp_line (start 4.05 -1.8) (end -2.05 -1.8) (layer F.SilkS) (width 0.12))
  (fp_line (start 0.5 -1.8) (end 0.5 -1.2) (layer F.SilkS) (width 0.12))
  (fp_line (start 0.5 -1.2) (end -1.45 -1.2) (layer F.SilkS) (width 0.12))
  (fp_line (start -1.45 -1.2) (end -1.45 2.3) (layer F.SilkS) (width 0.12))
  (fp_line (start -1.45 2.3) (end 3.45 2.3) (layer F.SilkS) (width 0.12))
  (fp_line (start 3.45 2.3) (end 3.45 -1.2) (layer F.SilkS) (width 0.12))
  (fp_line (start 3.45 -1.2) (end 1.5 -1.2) (layer F.SilkS) (width 0.12))
  (fp_line (start 1.5 -1.2) (end 1.5 -1.8) (layer F.SilkS) (width 0.12))
  (fp_line (start -2.05 -0.5) (end -1.45 -0.5) (layer F.SilkS) (width 0.12))
  (fp_line (start -2.05 0.8) (end -1.45 0.8) (layer F.SilkS) (width 0.12))
  (fp_line (start 4.05 -0.5) (end 3.45 -0.5) (layer F.SilkS) (width 0.12))
  (fp_line (start 4.05 0.8) (end 3.45 0.8) (layer F.SilkS) (width 0.12))
  (fp_line (start -0.3 -1.8) (end -0.3 -2) (layer F.SilkS) (width 0.12))
  (fp_line (start -0.3 -2) (end -0.6 -2) (layer F.SilkS) (width 0.12))
  (fp_line (start -0.6 -2) (end -0.6 -1.8) (layer F.SilkS) (width 0.12))
  (fp_line (start -0.3 -1.9) (end -0.6 -1.9) (layer F.SilkS) (width 0.12))
  (fp_line (start 0.9 2.3) (end 0.9 1.8) (layer F.SilkS) (width 0.12))
  (fp_line (start 0.9 1.8) (end 1.1 1.8) (layer F.SilkS) (width 0.12))
  (fp_line (start 1.1 1.8) (end 1.1 2.3) (layer F.SilkS) (width 0.12))
  (fp_line (start 1 2.3) (end 1 1.8) (layer F.SilkS) (width 0.12))
  (fp_line (start -1.1 -2.1) (end -2.35 -2.1) (layer F.SilkS) (width 0.12))
  (fp_line (start -2.35 -2.1) (end -2.35 -0.85) (layer F.SilkS) (width 0.12))
  (pad 1 thru_hole rect (at 0 0) (size 1.2 1.7) (drill 0.7) (layers *.Cu *.Mask) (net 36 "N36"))
  (pad 2 thru_hole oval (at 2 0) (size 1.2 1.7) (drill 0.7) (layers *.Cu *.Mask) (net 1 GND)))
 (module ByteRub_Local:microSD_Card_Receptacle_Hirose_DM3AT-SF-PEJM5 (layer F.Cu) (at 113.5 112)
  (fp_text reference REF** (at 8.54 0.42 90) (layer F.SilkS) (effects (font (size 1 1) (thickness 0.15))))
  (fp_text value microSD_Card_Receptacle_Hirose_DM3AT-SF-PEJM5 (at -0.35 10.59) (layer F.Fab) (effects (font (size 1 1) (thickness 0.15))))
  (fp_line (start -5.87 8.68) (end -4.03 8.68) (layer F.SilkS) (width 0.12))
  (fp_line (start 5.37 8.68) (end 3.14 8.68) (layer F.SilkS) (width 0.12))
  (fp_line (start -7.02 -7.83) (end -7.02 -7.32) (layer F.SilkS) (width 0.12))
  (fp_line (start -6.7 -7.83) (end -7.02 -7.83) (layer F.SilkS) (width 0.12))
  (fp_line (start 7.21 -7.83) (end 7.21 -5.92) (layer F.SilkS) (width 0.12))
  (fp_line (start 5.68 -7.83) (end 7.21 -7.83) (layer F.SilkS) (width 0.12))
  (pad 9 smd rect (at -5.8 -7.55) (size 0.7 1.2) (layers F.Cu F.Paste F.Mask))
  (pad 8 smd rect (at -4.85 -7.55) (size 0.7 1.2) (layers F.Cu F.Paste F.Mask))
  (pad 1 smd rect (at 2.85 -7.55) (size 0.7 1.2) (layers F.Cu F.Paste F.Mask))
  (pad 2 smd rect (at 1.75 -7.55) (size 0.7 1.2) (layers F.Cu F.Paste F.Mask))
  (pad 3 smd rect (at 0.65 -7.55) (size 0.7 1.2) (layers F.Cu F.Paste F.Mask))
  (pad 4 smd rect (at -0.45 -7.55) (size 0.7 1.2) (layers F.Cu F.Paste F.Mask))
  (pad 5 smd rect (at -1.55 -7.55) (size 0.7 1.2) (layers F.Cu F.Paste F.Mask))
  (pad 6 smd rect (at -2.65 -7.55) (size 0.7 1.2) (layers F.Cu F.Paste F.Mask))
  (pad 7 smd rect (at -3.75 -7.55) (size 0.7 1.2) (layers F.Cu F.Paste F.Mask))
  (pad 11 smd rect (at 4.4 -7.55) (size 1 1.2) (layers F.Cu F.Paste F.Mask))
  (pad 11 smd rect (at -6.75 -3.25) (size 1 1.2) (layers F.Cu F.Paste F.Mask))
  (pad 10 smd rect (at -6.75 2.95) (size 1 0.8) (layers F.Cu F.Paste F.Mask))
  (pad 11 smd rect (at -6.75 7.1) (size 1 2.8) (layers F.Cu F.Paste F.Mask))
  (pad 11 smd rect (at 6.75 7.55) (size 1.3 1.9) (layers F.Cu F.Paste F.Mask)))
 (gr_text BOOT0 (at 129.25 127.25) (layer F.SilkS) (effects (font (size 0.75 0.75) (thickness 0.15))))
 (gr_line (start 101 70) (end 100 71) (angle 90) (layer Edge.Cuts) (width 0.15))
 (gr_line (start 101 68) (end 101 70) (angle 90) (layer Edge.Cuts) (width 0.15))
 (gr_line (start 100 67) (end 101 68) (angle 90) (layer Edge.Cuts) (width 0.15))
 (gr_line (start 100 65.5) (end 100 67) (angle 90) (layer Edge.Cuts) (width 0.15))
 (gr_line (start 116 64) (end 101.5 64) (angle 90) (layer Edge.Cuts) (width 0.15))
 (gr_line (start 119 65.5) (end 116 64) (angle 90) (layer Edge.Cuts) (width 0.15))
 (gr_line (start 137.34 64) (end 134.34 65.5) (angle 90) (layer Edge.Cuts) (width 0.15))
 (gr_line (start 119 65.5) (end 134.34 65.5) (angle 90) (layer Edge.Cuts) (width 0.15))
 (gr_arc (start 101.5 65.5) (end 100 65.5) (angle 90) (layer Edge.Cuts) (width 0.15))
 (gr_arc (start 151.84 65.5) (end 151.84 64) (angle 90) (layer Edge.Cuts) (width 0.15))
 (gr_arc (start 151.84 126.5) (end 153.34 126.5) (angle 90) (layer Edge.Cuts) (width 0.15))
 (gr_arc (start 101.5 126.5) (end 101.5 128) (angle 90) (layer Edge.Cuts) (width 0.15))
 (gr_line (start 151.84 64) (end 137.34 64) (angle 90) (layer Edge.Cuts) (width 0.15))
 (gr_line (start 153.34 126.5) (end 153.34 65.5) (angle 90) (layer Edge.Cuts) (width 0.15))
 (gr_line (start 101.5 128) (end 151.84 128) (angle 90) (layer Edge.Cuts) (width 0.15))
 (gr_line (start 100 71) (end 100 126.5) (angle 90) (layer Edge.Cuts) (width 0.15))
 (segment (start 149 77.2) (end 148.8 77) (width 0.1524) (layer F.Cu) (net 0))
 (segment (start 124.49 117.84) (end 125.4 117.84) (width 0.1524) (layer B.Cu) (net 1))
 (segment (start 125.4 117.84) (end 126.56 117.84) (width 0.1524) (layer F.Cu) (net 1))
 (segment (start 130.48 125.46) (end 130.48 125.18) (width 0.1524) (layer F.Cu) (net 20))
 (segment (start 127.94 125.46) (end 128.29 125.46) (width 0.1524) (layer B.Cu) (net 34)))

